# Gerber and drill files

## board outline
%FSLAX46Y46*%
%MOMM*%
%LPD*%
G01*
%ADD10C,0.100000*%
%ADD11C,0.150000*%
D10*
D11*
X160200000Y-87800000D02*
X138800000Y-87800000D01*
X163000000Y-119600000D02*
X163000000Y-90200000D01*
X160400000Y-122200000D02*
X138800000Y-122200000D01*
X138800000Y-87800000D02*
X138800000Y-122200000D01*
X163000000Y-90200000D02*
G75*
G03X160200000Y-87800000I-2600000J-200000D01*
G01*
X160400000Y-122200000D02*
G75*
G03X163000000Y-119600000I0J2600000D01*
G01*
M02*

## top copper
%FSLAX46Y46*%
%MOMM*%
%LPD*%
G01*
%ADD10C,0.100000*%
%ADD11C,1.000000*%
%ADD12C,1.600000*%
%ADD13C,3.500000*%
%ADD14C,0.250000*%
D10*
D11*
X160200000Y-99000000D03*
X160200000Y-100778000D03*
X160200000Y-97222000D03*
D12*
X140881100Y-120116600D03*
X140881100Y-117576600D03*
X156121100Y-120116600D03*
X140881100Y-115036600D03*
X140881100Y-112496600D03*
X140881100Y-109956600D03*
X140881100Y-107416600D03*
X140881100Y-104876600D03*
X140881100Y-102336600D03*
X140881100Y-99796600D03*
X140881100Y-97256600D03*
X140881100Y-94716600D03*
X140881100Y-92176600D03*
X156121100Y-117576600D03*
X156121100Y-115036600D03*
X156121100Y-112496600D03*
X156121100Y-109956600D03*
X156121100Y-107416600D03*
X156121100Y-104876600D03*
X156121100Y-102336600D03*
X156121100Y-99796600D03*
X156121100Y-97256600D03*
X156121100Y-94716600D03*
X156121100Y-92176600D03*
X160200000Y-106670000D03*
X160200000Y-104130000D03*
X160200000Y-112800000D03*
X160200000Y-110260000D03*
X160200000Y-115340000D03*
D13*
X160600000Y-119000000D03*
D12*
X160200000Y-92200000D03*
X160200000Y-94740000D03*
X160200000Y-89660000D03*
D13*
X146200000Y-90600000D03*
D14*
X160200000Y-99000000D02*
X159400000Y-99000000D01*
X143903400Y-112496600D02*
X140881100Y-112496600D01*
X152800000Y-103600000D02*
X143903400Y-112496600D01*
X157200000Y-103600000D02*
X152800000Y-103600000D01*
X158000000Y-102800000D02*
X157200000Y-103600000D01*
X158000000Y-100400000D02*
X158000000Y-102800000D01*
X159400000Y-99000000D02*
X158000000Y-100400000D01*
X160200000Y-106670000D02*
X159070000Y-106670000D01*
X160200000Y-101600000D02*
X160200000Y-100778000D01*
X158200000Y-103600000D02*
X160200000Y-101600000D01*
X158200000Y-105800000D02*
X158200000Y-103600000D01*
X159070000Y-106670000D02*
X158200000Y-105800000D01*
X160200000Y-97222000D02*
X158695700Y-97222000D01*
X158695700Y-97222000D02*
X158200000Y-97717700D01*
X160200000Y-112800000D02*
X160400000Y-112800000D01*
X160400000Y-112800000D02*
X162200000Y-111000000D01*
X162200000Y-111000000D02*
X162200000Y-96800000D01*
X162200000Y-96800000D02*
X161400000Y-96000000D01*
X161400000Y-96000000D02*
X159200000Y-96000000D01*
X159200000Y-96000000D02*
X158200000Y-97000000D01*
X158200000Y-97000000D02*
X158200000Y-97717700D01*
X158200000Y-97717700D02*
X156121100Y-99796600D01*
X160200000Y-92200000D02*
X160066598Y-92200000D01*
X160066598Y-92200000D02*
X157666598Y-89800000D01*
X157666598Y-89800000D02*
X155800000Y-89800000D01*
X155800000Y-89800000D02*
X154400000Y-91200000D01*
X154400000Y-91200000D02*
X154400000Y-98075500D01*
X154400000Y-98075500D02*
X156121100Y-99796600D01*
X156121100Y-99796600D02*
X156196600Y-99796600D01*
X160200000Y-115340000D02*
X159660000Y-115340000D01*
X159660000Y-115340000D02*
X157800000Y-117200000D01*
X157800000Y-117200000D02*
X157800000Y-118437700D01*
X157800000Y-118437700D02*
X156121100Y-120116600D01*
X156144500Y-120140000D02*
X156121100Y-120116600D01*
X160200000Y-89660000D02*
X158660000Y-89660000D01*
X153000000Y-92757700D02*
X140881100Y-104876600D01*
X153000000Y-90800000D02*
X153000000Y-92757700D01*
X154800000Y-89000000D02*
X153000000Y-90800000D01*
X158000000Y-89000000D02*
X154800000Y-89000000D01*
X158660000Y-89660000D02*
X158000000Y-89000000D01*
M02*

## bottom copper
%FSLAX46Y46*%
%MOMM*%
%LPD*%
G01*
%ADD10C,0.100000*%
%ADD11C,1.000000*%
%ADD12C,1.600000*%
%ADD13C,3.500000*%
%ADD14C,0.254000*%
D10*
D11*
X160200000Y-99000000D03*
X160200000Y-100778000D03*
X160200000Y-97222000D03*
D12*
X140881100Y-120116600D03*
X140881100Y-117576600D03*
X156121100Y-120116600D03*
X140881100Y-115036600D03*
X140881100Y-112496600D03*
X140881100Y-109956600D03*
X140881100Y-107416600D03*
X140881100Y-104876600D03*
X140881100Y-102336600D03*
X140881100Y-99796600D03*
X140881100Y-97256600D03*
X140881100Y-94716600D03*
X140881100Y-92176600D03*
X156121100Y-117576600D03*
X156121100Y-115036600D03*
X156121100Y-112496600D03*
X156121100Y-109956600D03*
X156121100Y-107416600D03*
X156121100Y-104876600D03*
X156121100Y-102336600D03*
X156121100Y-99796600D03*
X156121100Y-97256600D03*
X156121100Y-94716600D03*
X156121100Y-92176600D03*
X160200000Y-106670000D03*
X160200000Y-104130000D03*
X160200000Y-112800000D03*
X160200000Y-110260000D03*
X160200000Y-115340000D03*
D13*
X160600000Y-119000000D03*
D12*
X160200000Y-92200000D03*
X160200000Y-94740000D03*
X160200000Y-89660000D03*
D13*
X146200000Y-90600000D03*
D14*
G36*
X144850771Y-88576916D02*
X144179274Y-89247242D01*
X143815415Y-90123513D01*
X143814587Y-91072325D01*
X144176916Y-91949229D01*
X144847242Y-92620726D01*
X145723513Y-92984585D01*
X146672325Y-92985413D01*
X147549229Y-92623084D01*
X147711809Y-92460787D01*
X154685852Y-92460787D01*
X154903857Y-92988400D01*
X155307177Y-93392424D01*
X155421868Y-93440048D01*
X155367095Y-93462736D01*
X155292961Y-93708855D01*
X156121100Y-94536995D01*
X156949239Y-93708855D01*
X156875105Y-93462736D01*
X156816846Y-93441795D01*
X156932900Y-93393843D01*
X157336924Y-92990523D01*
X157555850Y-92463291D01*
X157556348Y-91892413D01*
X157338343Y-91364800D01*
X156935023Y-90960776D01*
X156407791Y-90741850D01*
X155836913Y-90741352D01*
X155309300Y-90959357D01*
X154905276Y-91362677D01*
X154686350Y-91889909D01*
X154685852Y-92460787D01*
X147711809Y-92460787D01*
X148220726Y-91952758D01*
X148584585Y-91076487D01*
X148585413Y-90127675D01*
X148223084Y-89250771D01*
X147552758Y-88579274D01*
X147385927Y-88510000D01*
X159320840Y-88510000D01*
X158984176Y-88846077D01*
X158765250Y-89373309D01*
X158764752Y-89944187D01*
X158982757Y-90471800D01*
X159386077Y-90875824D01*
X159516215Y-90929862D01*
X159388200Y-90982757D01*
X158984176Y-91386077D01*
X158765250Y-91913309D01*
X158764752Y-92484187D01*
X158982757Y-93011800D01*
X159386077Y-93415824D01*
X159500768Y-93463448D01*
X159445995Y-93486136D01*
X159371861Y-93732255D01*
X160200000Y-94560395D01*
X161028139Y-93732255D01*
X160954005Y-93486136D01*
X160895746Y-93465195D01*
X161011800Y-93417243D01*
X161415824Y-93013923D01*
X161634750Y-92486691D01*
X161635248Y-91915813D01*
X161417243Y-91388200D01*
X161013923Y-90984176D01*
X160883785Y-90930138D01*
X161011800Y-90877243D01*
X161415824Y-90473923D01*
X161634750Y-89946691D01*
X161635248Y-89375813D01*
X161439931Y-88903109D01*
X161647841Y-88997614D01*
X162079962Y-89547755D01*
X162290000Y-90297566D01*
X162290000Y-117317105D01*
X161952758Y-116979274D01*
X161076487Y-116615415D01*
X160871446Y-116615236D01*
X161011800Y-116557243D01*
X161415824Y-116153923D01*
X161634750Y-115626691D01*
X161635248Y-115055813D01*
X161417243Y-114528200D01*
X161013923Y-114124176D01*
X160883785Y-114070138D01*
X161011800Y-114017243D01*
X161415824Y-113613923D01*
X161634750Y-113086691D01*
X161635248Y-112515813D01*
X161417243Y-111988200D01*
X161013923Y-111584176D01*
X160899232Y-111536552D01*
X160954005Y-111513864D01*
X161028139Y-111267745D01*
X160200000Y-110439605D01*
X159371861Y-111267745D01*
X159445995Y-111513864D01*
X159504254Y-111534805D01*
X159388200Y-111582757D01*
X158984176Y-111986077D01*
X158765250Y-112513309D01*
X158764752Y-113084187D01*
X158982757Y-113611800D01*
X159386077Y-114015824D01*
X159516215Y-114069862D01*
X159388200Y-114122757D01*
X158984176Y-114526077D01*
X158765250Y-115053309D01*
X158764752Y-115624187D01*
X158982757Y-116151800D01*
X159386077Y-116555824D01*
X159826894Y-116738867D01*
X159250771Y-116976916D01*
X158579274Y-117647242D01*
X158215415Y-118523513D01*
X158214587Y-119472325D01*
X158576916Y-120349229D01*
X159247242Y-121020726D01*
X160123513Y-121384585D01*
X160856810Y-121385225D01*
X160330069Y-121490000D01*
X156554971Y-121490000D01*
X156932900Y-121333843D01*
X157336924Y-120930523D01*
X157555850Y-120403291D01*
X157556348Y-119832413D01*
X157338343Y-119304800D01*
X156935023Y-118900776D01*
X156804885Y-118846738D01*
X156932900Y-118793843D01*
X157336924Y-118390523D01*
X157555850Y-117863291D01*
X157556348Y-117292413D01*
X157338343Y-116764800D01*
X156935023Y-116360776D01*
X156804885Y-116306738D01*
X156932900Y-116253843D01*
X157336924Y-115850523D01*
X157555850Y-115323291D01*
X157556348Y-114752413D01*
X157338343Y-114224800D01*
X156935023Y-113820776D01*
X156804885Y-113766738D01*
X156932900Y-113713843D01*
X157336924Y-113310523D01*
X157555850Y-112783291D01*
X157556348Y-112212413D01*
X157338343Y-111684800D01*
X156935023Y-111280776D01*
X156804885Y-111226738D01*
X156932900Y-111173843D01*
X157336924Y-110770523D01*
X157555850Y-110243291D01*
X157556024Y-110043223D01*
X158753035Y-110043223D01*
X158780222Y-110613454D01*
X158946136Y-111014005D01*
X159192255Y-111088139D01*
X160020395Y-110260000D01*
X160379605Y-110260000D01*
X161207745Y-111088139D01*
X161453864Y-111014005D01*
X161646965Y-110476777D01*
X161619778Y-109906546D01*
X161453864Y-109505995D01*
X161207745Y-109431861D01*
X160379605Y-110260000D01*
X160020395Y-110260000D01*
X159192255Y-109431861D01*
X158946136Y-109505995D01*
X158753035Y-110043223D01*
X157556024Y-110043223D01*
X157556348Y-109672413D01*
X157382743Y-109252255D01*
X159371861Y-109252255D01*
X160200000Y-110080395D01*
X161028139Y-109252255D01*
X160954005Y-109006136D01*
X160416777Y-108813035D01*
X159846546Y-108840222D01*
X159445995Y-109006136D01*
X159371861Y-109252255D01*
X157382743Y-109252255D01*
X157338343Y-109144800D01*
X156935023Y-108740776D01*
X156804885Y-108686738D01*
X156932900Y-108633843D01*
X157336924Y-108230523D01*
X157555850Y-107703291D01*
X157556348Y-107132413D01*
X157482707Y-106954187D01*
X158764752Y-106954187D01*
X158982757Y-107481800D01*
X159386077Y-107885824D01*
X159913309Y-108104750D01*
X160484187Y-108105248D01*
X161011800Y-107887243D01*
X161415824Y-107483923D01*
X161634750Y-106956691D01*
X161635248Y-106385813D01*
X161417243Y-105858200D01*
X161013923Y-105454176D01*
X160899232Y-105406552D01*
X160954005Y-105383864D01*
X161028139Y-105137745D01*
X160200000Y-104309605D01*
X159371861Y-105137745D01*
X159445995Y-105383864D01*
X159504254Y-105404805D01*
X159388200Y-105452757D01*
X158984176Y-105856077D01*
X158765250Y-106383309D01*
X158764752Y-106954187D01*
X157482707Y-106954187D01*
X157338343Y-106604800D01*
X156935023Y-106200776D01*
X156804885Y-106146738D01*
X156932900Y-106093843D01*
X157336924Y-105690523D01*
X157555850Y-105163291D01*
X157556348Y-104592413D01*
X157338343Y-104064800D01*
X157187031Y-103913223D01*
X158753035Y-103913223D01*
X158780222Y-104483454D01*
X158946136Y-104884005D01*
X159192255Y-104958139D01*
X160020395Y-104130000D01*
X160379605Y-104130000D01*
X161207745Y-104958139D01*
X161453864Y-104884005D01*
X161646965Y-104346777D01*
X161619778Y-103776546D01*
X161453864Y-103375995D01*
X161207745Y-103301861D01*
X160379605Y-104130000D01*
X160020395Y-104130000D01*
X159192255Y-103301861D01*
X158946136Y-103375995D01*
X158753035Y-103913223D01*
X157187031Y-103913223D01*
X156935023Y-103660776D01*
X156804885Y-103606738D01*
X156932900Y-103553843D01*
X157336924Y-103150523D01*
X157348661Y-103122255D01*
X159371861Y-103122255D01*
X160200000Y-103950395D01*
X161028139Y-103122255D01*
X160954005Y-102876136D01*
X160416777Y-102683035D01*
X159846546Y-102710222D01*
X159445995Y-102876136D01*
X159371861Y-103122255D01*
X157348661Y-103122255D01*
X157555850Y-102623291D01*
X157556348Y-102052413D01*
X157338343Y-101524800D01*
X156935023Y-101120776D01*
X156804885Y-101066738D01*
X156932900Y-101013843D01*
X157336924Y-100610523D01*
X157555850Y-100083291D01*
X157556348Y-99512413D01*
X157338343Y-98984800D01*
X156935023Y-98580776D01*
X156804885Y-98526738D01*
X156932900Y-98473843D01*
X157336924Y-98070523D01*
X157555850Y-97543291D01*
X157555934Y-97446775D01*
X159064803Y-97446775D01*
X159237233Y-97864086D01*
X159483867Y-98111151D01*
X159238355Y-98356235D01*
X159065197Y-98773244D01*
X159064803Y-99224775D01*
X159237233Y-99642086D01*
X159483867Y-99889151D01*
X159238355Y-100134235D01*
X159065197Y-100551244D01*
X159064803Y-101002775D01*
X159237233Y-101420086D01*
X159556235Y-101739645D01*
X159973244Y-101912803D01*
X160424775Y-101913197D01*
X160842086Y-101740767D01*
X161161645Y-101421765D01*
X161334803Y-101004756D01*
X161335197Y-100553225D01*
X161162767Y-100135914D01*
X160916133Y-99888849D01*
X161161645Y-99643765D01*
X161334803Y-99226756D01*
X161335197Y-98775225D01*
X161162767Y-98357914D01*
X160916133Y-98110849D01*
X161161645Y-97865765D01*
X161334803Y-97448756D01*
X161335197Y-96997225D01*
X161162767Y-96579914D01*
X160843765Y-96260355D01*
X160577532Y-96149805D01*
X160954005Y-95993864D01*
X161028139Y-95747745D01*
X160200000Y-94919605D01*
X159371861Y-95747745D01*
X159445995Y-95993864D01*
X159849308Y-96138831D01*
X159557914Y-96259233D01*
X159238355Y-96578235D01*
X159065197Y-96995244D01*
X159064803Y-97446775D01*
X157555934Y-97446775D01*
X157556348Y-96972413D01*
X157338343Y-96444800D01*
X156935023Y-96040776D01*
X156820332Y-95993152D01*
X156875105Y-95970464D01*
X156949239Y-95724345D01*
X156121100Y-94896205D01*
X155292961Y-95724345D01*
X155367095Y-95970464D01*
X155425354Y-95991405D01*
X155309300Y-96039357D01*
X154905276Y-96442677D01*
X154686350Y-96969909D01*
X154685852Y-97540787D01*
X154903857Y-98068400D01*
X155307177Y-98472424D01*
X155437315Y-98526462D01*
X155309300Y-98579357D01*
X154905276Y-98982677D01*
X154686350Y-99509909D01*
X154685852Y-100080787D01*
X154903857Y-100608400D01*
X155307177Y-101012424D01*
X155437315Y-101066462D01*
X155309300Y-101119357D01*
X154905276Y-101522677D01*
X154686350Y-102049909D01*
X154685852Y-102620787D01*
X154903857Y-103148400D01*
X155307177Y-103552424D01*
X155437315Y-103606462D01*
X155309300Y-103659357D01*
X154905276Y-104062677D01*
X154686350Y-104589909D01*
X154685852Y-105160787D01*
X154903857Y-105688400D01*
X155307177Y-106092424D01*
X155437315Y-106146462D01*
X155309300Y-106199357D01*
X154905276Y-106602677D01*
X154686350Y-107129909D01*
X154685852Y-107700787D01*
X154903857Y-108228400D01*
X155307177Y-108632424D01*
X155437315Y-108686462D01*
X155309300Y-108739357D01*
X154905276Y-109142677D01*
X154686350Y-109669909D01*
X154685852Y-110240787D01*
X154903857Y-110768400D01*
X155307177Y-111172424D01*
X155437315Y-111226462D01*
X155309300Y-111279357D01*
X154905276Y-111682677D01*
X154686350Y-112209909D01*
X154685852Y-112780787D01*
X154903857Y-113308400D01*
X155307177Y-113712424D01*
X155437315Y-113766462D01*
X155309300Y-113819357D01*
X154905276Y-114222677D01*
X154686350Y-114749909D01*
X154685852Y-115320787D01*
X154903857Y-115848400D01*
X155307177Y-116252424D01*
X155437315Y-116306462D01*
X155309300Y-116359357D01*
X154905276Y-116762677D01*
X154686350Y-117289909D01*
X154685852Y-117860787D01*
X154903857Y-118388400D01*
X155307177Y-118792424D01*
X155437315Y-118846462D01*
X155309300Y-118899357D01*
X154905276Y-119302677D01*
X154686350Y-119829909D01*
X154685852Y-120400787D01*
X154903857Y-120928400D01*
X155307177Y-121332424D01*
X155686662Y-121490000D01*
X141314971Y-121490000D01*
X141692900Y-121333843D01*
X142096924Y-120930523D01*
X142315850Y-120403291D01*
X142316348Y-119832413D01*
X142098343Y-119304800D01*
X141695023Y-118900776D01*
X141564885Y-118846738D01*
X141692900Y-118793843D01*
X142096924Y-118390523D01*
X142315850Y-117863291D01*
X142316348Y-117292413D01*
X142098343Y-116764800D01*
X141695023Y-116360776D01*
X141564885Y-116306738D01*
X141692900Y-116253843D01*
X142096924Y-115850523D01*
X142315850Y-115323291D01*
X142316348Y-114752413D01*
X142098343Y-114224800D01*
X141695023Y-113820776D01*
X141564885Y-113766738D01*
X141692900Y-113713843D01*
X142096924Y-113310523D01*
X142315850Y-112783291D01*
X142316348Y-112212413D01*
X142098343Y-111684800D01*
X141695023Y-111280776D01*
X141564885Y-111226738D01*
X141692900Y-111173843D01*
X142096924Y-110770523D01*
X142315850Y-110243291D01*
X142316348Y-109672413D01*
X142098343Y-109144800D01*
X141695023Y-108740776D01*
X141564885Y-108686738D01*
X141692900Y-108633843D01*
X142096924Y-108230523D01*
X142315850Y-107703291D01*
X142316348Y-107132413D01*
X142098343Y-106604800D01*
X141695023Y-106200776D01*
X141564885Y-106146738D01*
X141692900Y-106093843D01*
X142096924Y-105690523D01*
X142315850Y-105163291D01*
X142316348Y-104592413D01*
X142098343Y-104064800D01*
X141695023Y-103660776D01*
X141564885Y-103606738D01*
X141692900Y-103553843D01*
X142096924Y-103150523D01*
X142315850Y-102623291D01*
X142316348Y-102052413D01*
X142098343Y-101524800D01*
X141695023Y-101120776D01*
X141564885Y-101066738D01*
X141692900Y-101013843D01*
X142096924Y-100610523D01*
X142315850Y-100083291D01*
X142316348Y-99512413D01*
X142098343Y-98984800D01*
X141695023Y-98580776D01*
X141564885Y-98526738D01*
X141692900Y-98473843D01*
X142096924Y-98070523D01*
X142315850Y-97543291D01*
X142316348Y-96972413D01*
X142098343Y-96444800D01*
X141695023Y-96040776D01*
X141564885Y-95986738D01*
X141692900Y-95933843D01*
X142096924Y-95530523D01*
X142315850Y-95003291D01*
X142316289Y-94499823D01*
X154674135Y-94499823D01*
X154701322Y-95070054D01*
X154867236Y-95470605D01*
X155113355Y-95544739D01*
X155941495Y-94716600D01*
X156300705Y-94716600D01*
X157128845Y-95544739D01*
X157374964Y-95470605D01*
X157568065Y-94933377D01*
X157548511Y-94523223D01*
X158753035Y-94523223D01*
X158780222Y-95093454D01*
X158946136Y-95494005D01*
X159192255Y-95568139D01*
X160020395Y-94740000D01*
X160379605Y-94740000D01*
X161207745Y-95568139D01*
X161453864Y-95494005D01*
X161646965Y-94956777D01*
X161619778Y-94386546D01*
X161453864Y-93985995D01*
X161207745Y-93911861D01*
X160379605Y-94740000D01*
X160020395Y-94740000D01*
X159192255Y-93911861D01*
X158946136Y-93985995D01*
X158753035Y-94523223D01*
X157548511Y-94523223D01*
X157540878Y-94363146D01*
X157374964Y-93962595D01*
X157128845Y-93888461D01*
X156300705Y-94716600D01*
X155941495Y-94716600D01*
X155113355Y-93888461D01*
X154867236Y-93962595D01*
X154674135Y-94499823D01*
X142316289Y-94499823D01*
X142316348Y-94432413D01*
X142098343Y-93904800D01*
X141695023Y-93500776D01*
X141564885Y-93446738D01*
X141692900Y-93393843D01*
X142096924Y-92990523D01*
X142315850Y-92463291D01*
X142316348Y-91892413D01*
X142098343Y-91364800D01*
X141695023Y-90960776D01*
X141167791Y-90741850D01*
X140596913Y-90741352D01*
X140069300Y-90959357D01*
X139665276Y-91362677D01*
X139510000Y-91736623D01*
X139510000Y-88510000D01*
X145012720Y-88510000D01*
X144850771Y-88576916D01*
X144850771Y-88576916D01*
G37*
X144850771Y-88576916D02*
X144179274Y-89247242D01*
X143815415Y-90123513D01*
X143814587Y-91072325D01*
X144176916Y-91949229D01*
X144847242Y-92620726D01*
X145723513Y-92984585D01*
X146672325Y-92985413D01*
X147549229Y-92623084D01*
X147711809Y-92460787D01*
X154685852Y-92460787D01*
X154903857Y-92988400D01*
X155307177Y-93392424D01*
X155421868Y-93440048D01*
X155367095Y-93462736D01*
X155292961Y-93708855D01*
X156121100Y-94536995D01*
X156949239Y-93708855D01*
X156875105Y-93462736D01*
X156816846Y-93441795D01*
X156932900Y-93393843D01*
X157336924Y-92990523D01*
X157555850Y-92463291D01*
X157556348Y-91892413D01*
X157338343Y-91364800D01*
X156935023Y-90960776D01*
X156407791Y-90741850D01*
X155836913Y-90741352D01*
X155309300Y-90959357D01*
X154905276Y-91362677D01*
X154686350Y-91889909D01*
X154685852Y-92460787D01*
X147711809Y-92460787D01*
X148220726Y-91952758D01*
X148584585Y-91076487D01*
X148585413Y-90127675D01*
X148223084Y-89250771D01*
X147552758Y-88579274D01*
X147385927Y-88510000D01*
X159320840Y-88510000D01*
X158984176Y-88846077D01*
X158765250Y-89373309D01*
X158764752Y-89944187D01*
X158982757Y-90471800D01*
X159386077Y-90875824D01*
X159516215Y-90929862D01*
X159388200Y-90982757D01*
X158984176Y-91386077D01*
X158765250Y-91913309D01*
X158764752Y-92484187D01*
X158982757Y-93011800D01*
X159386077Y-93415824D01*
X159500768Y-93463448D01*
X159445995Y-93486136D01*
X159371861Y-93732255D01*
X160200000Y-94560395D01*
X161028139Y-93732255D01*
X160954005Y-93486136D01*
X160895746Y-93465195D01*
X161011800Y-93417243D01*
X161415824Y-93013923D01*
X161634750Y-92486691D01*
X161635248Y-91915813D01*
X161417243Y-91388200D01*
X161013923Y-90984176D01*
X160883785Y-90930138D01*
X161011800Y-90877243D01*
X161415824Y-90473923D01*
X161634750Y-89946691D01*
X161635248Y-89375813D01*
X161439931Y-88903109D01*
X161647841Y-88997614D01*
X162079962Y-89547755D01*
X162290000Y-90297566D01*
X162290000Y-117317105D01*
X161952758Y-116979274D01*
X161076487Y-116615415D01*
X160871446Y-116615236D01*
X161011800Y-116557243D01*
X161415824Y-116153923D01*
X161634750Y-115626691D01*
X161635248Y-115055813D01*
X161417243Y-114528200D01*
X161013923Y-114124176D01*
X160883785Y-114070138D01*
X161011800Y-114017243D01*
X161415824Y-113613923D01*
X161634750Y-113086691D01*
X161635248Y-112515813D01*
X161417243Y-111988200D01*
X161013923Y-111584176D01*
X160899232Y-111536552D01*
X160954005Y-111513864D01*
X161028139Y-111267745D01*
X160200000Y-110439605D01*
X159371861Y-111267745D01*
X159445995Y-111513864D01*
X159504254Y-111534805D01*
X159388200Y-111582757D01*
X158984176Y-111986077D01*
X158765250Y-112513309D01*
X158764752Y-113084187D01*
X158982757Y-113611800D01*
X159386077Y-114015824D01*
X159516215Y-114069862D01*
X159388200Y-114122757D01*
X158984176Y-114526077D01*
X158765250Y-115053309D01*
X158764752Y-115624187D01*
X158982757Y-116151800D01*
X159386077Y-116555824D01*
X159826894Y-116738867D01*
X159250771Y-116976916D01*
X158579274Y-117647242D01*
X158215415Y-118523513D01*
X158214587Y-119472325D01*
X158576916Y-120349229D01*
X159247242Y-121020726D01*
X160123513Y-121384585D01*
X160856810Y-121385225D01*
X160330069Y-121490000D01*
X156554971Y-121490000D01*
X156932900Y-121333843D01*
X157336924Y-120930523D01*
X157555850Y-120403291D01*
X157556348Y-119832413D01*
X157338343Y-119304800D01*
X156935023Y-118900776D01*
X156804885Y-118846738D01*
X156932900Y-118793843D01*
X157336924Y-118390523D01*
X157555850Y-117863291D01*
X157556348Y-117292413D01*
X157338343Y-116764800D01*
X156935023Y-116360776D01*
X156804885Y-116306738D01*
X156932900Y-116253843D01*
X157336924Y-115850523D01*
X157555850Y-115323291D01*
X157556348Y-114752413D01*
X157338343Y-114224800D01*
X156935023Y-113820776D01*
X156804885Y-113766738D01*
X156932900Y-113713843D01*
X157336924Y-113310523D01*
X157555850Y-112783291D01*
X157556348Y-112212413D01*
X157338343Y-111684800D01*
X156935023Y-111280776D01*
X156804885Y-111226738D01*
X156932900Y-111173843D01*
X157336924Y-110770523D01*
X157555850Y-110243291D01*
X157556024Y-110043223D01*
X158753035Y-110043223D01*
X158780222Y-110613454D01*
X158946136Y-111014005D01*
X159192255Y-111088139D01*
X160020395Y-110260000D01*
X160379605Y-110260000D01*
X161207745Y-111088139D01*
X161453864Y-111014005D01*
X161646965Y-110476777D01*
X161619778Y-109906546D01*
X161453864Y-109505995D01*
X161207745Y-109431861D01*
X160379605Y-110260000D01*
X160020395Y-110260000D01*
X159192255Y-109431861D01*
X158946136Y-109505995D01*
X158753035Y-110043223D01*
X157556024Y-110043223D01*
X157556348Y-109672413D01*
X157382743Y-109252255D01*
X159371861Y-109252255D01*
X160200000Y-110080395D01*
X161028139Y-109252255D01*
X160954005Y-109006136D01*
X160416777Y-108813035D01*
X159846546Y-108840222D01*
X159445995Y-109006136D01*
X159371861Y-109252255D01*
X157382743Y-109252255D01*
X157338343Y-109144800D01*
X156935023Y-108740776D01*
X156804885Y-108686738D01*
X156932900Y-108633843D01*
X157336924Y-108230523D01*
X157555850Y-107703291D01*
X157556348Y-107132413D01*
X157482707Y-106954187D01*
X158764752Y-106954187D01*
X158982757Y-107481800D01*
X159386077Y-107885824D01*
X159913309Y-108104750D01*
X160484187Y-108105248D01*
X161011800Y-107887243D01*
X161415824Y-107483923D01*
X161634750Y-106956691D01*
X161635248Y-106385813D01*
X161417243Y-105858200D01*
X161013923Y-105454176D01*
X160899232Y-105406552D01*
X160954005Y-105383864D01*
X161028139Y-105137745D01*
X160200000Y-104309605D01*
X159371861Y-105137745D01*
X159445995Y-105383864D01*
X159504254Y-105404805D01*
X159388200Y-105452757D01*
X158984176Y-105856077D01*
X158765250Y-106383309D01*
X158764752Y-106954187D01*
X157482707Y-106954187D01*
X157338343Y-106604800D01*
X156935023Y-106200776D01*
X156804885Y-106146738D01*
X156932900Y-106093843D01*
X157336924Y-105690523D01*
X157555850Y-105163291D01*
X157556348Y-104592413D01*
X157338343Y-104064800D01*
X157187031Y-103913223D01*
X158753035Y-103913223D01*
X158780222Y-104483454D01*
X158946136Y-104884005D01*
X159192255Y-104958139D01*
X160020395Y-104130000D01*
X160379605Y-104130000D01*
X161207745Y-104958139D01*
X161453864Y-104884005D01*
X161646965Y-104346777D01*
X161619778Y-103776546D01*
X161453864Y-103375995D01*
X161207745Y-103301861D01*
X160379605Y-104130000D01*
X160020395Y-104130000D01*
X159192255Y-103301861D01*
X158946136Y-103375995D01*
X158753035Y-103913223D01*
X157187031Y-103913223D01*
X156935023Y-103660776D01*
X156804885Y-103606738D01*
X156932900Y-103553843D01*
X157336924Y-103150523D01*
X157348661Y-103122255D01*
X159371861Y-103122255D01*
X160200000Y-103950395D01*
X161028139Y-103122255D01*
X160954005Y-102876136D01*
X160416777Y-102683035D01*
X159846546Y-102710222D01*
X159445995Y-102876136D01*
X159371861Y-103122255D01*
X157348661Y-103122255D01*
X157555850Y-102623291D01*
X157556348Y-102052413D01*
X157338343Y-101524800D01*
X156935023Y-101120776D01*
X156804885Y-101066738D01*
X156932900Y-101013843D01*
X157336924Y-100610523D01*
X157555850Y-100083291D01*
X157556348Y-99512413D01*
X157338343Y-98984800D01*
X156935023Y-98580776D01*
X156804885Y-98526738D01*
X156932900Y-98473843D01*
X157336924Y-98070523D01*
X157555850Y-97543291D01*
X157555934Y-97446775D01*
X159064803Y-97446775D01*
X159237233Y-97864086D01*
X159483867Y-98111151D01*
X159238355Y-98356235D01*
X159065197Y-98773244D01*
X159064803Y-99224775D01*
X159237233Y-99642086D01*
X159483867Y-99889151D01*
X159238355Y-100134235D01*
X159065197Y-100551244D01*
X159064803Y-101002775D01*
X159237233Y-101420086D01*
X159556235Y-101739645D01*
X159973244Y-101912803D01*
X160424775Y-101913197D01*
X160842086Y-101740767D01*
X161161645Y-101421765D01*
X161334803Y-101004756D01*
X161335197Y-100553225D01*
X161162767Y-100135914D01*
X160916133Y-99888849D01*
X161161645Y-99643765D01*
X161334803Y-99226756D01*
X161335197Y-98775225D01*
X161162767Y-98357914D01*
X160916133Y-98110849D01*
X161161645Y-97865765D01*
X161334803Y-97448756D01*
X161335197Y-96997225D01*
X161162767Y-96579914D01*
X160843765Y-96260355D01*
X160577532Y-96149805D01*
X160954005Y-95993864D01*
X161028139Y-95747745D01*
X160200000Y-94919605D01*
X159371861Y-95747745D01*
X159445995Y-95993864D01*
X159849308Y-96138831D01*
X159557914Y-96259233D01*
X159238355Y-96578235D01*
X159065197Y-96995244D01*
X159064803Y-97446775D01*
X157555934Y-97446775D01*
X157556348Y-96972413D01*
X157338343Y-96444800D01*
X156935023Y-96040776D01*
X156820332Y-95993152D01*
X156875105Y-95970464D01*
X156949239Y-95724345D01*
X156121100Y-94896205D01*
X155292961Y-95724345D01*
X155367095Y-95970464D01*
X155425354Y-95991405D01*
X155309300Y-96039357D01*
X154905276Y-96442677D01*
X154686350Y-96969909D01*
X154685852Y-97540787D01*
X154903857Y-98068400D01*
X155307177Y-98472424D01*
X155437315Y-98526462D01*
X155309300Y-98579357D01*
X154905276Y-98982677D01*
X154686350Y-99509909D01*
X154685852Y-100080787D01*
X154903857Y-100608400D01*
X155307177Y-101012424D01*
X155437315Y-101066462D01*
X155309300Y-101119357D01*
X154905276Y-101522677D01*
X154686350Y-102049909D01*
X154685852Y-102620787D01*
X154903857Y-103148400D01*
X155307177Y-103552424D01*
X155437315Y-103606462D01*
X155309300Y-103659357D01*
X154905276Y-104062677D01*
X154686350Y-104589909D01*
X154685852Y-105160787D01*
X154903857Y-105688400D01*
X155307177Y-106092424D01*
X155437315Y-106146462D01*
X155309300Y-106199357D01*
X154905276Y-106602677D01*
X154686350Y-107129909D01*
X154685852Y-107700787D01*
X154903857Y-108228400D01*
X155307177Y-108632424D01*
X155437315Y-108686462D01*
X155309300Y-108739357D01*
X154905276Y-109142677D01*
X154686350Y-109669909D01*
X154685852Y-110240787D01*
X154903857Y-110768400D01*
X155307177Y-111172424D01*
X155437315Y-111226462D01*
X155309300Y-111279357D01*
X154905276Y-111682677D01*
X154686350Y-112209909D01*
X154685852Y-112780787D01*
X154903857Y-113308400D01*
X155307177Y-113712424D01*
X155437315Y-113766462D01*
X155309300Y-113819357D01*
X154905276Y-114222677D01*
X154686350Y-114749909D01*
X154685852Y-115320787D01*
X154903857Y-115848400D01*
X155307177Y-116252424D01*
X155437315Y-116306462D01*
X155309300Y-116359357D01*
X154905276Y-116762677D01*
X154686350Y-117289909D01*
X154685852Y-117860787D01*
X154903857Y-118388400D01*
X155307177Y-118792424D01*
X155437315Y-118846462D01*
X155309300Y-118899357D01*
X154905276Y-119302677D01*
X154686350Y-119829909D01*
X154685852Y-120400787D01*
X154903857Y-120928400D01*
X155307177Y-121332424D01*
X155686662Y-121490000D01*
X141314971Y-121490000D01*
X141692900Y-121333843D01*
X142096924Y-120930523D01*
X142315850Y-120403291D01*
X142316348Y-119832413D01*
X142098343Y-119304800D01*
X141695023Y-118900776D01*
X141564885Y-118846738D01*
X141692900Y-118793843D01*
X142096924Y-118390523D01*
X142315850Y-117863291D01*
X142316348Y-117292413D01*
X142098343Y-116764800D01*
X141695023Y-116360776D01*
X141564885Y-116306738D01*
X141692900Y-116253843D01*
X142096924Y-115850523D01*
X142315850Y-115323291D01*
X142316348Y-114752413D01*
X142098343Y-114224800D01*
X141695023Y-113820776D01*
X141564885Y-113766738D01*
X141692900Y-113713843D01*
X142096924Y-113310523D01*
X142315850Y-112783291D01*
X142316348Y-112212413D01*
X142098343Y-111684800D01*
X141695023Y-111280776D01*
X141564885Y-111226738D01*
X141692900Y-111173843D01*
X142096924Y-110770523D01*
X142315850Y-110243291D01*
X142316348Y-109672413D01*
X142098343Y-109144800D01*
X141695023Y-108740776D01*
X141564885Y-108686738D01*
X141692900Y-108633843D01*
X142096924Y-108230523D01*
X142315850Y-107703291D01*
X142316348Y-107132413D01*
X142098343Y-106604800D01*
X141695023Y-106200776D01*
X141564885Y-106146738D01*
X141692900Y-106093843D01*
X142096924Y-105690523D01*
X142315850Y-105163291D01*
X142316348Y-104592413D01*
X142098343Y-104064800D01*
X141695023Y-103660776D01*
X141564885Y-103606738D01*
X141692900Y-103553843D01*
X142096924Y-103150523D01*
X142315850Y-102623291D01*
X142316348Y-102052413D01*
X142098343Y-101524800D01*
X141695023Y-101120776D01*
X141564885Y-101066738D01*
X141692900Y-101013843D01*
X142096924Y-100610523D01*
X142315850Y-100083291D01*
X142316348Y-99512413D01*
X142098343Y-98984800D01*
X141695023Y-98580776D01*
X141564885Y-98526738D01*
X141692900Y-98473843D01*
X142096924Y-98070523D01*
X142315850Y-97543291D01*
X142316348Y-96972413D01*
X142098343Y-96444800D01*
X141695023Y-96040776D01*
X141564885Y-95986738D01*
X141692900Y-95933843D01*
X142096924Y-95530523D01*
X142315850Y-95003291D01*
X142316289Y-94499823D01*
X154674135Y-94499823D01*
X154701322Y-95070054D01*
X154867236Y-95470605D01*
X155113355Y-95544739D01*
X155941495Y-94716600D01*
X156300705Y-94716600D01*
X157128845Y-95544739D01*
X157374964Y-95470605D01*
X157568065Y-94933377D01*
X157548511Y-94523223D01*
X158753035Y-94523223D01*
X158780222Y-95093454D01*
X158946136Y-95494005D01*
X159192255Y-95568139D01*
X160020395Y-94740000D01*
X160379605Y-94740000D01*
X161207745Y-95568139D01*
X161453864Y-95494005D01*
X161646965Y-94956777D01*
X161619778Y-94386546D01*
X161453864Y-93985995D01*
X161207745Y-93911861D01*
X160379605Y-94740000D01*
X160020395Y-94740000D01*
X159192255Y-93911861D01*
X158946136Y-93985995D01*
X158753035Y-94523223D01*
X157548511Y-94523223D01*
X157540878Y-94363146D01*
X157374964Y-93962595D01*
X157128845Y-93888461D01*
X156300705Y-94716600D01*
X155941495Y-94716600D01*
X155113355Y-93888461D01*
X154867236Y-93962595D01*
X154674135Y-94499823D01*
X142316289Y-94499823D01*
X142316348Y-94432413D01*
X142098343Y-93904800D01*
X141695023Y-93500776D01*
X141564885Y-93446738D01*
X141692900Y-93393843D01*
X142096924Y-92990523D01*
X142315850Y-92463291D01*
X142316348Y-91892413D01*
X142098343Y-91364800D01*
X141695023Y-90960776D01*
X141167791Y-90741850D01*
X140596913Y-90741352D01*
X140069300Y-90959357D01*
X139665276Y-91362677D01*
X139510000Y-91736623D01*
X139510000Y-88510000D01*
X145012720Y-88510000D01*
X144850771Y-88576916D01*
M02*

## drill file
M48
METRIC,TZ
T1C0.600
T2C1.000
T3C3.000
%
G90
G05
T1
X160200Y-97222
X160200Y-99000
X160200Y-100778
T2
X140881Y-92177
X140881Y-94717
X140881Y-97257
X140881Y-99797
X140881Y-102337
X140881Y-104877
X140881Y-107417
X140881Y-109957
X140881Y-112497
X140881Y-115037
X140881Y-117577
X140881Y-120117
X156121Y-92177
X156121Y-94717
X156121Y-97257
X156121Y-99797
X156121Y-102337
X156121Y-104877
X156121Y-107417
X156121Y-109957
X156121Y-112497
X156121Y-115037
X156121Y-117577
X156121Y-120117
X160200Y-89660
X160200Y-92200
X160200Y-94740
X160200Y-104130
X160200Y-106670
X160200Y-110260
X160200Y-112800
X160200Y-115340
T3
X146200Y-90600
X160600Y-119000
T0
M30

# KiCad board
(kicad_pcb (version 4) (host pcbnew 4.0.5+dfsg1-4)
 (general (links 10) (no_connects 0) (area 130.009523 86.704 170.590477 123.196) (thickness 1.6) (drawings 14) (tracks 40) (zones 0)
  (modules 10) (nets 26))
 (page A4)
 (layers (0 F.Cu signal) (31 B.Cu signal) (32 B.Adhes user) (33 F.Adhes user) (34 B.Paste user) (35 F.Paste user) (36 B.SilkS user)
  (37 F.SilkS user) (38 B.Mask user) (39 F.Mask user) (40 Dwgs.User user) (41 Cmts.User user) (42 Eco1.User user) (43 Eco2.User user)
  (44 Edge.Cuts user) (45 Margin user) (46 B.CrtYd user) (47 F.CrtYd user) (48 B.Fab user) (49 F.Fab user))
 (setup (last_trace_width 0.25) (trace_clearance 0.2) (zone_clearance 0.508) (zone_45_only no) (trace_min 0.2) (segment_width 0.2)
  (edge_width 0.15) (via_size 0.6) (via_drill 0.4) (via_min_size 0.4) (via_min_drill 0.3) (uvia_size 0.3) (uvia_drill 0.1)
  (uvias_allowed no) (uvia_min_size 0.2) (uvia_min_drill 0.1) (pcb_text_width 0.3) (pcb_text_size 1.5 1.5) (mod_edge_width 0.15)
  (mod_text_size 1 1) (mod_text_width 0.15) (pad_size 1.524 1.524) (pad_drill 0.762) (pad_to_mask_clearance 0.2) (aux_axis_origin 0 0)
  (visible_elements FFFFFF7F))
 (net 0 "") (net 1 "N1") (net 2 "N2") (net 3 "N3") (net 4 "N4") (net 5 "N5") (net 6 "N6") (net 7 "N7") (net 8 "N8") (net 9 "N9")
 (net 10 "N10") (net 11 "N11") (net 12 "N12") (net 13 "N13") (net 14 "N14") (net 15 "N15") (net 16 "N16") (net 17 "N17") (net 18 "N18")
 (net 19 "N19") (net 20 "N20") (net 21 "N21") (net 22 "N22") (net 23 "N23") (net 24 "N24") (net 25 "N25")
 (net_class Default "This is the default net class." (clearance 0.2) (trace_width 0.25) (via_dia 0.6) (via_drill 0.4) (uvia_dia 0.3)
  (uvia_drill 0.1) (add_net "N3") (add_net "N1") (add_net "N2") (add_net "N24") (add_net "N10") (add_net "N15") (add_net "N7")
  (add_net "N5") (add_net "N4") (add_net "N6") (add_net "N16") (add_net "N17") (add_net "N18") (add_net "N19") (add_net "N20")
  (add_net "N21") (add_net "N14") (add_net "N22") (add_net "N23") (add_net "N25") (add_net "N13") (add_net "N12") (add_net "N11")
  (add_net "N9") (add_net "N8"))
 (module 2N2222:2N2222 (layer F.Cu) (at 160.2 99 270)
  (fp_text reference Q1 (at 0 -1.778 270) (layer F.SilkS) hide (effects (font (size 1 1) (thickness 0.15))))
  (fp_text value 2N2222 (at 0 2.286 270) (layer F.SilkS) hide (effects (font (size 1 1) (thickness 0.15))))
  (pad 2 thru_hole circle (at 0 0 270) (size 1 1) (drill 0.6) (layers *.Cu *.Mask F.SilkS) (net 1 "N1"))
  (pad 3 thru_hole circle (at 1.778 0 270) (size 1 1) (drill 0.6) (layers *.Cu *.Mask F.SilkS) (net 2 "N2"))
  (pad 1 thru_hole circle (at -1.778 0 270) (size 1 1) (drill 0.6) (layers *.Cu *.Mask F.SilkS) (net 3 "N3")))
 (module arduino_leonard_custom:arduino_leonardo (layer F.Cu) (at 148.5011 105.0036)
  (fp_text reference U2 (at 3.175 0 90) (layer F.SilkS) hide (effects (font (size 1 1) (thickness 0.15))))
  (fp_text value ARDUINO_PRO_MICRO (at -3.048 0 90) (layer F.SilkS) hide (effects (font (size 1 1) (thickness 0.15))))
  (pad 12 thru_hole circle (at -7.62 15.113) (size 1.6 1.6) (drill 1) (layers *.Cu *.Mask F.SilkS) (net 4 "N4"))
  (pad 11 thru_hole circle (at -7.62 12.573) (size 1.6 1.6) (drill 1) (layers *.Cu *.Mask F.SilkS) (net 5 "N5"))
  (pad 13 thru_hole circle (at 7.62 15.113) (size 1.6 1.6) (drill 1) (layers *.Cu *.Mask F.SilkS) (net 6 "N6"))
  (pad 10 thru_hole circle (at -7.62 10.033) (size 1.6 1.6) (drill 1) (layers *.Cu *.Mask F.SilkS) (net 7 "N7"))
  (pad 9 thru_hole circle (at -7.62 7.493) (size 1.6 1.6) (drill 1) (layers *.Cu *.Mask F.SilkS) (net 1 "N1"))
  (pad 8 thru_hole circle (at -7.62 4.953) (size 1.6 1.6) (drill 1) (layers *.Cu *.Mask F.SilkS) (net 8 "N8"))
  (pad 7 thru_hole circle (at -7.62 2.413) (size 1.6 1.6) (drill 1) (layers *.Cu *.Mask F.SilkS) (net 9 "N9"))
  (pad 6 thru_hole circle (at -7.62 -0.127) (size 1.6 1.6) (drill 1) (layers *.Cu *.Mask F.SilkS) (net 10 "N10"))
  (pad 5 thru_hole circle (at -7.62 -2.667) (size 1.6 1.6) (drill 1) (layers *.Cu *.Mask F.SilkS) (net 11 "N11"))
  (pad 4 thru_hole circle (at -7.62 -5.207) (size 1.6 1.6) (drill 1) (layers *.Cu *.Mask F.SilkS) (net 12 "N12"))
  (pad 3 thru_hole circle (at -7.62 -7.747) (size 1.6 1.6) (drill 1) (layers *.Cu *.Mask F.SilkS) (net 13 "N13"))
  (pad 2 thru_hole circle (at -7.62 -10.287) (size 1.6 1.6) (drill 1) (layers *.Cu *.Mask F.SilkS) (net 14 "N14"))
  (pad 1 thru_hole circle (at -7.62 -12.827) (size 1.6 1.6) (drill 1) (layers *.Cu *.Mask F.SilkS) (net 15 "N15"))
  (pad 14 thru_hole circle (at 7.62 12.573) (size 1.6 1.6) (drill 1) (layers *.Cu *.Mask F.SilkS) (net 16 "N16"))
  (pad 15 thru_hole circle (at 7.62 10.033) (size 1.6 1.6) (drill 1) (layers *.Cu *.Mask F.SilkS) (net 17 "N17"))
  (pad 16 thru_hole circle (at 7.62 7.493) (size 1.6 1.6) (drill 1) (layers *.Cu *.Mask F.SilkS) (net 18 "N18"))
  (pad 17 thru_hole circle (at 7.62 4.953) (size 1.6 1.6) (drill 1) (layers *.Cu *.Mask F.SilkS) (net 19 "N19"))
  (pad 18 thru_hole circle (at 7.62 2.413) (size 1.6 1.6) (drill 1) (layers *.Cu *.Mask F.SilkS) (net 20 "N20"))
  (pad 19 thru_hole circle (at 7.62 -0.127) (size 1.6 1.6) (drill 1) (layers *.Cu *.Mask F.SilkS) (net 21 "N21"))
  (pad 20 thru_hole circle (at 7.62 -2.667) (size 1.6 1.6) (drill 1) (layers *.Cu *.Mask F.SilkS) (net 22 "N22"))
  (pad 21 thru_hole circle (at 7.62 -5.207) (size 1.6 1.6) (drill 1) (layers *.Cu *.Mask F.SilkS) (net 3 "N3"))
  (pad 22 thru_hole circle (at 7.62 -7.747) (size 1.6 1.6) (drill 1) (layers *.Cu *.Mask F.SilkS) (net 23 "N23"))
  (pad 23 thru_hole circle (at 7.62 -10.287) (size 1.6 1.6) (drill 1) (layers *.Cu *.Mask F.SilkS) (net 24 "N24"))
  (pad 24 thru_hole circle (at 7.62 -12.827) (size 1.6 1.6) (drill 1) (layers *.Cu *.Mask F.SilkS) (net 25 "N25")))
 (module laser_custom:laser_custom (layer F.Cu) (at 160.2 105.4 90)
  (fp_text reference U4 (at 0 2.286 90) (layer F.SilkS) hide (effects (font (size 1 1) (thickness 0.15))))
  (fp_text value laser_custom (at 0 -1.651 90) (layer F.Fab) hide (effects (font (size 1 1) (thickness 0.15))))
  (pad 1 thru_hole circle (at -1.27 0 90) (size 1.6 1.6) (drill 1) (layers *.Cu *.Mask) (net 2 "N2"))
  (pad 2 thru_hole circle (at 1.27 0 90) (size 1.6 1.6) (drill 1) (layers *.Cu *.Mask) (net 24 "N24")))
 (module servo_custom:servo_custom (layer F.Cu) (at 160.2 112.8 270)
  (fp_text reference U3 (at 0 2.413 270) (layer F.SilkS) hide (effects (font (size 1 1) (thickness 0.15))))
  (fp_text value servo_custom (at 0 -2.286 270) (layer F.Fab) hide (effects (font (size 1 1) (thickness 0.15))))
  (pad 2 thru_hole circle (at 0 0 270) (size 1.6 1.6) (drill 1) (layers *.Cu *.Mask) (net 3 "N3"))
  (pad 1 thru_hole circle (at -2.54 0 270) (size 1.6 1.6) (drill 1) (layers *.Cu *.Mask) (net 24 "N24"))
  (pad 3 thru_hole circle (at 2.54 0 270) (size 1.6 1.6) (drill 1) (layers *.Cu *.Mask) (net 6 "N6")))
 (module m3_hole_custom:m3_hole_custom (layer F.Cu) (at 136.4 119.2)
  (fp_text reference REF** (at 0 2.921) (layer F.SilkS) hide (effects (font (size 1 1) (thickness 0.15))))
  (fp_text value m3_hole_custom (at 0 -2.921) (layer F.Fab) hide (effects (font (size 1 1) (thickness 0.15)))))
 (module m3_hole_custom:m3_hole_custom (layer F.Cu) (at 164.2 90.6)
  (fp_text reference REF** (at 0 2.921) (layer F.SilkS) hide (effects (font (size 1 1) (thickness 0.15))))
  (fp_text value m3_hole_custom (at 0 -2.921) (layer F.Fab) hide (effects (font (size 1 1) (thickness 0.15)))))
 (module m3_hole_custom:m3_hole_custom (layer F.Cu) (at 136.4 90.6)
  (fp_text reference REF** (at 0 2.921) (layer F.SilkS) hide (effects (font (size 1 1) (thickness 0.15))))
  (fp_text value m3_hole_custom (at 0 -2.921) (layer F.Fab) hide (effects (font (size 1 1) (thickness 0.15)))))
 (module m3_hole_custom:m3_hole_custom (layer F.Cu) (at 160.6 119)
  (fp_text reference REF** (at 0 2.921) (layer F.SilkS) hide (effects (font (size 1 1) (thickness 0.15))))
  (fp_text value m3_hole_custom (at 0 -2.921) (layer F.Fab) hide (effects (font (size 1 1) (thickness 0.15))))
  (pad 1 thru_hole circle (at 0 0) (size 3.5 3.5) (drill 3) (layers *.Cu *.Mask)))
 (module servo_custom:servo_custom (layer F.Cu) (at 160.2 92.2 90)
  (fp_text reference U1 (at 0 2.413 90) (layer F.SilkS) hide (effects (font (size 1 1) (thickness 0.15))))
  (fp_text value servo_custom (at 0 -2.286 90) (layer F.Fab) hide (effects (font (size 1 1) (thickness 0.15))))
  (pad 2 thru_hole circle (at 0 0 90) (size 1.6 1.6) (drill 1) (layers *.Cu *.Mask) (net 3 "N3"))
  (pad 1 thru_hole circle (at -2.54 0 90) (size 1.6 1.6) (drill 1) (layers *.Cu *.Mask) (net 24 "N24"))
  (pad 3 thru_hole circle (at 2.54 0 90) (size 1.6 1.6) (drill 1) (layers *.Cu *.Mask) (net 10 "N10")))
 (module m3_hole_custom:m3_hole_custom (layer F.Cu) (at 146.2 90.6)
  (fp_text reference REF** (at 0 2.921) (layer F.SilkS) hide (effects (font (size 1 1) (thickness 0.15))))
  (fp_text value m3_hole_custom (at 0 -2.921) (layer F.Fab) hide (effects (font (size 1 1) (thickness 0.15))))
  (pad 1 thru_hole circle (at 0 0) (size 3.5 3.5) (drill 3) (layers *.Cu *.Mask)))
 (gr_line (start 160.2 87.8) (end 138.8 87.8) (angle 90) (layer Edge.Cuts) (width 0.15))
 (gr_line (start 163 119.6) (end 163 90.2) (angle 90) (layer Edge.Cuts) (width 0.15))
 (gr_line (start 160.4 122.2) (end 138.8 122.2) (angle 90) (layer Edge.Cuts) (width 0.15))
 (gr_line (start 138.8 87.8) (end 138.8 122.2) (angle 90) (layer Edge.Cuts) (width 0.15))
 (gr_arc (start 160.4 90.4) (end 160.2 87.8) (angle 90) (layer Edge.Cuts) (width 0.15))
 (gr_arc (start 160.4 119.6) (end 163 119.6) (angle 90) (layer Edge.Cuts) (width 0.15))
 (segment (start 160.2 99) (end 159.4 99) (width 0.25) (layer F.Cu) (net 1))
 (segment (start 143.9034 112.4966) (end 140.8811 112.4966) (width 0.25) (layer F.Cu) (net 1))
 (segment (start 152.8 103.6) (end 143.9034 112.4966) (width 0.25) (layer F.Cu) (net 1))
 (segment (start 157.2 103.6) (end 152.8 103.6) (width 0.25) (layer F.Cu) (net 1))
 (segment (start 158 102.8) (end 157.2 103.6) (width 0.25) (layer F.Cu) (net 1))
 (segment (start 158 100.4) (end 158 102.8) (width 0.25) (layer F.Cu) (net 1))
 (segment (start 159.4 99) (end 158 100.4) (width 0.25) (layer F.Cu) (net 1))
 (segment (start 160.2 106.67) (end 159.07 106.67) (width 0.25) (layer F.Cu) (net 2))
 (segment (start 160.2 101.6) (end 160.2 100.778) (width 0.25) (layer F.Cu) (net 2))
 (segment (start 158.2 103.6) (end 160.2 101.6) (width 0.25) (layer F.Cu) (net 2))
 (segment (start 158.2 105.8) (end 158.2 103.6) (width 0.25) (layer F.Cu) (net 2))
 (segment (start 159.07 106.67) (end 158.2 105.8) (width 0.25) (layer F.Cu) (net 2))
 (segment (start 160.2 97.222) (end 158.6957 97.222) (width 0.25) (layer F.Cu) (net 3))
 (segment (start 158.6957 97.222) (end 158.2 97.7177) (width 0.25) (layer F.Cu) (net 3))
 (segment (start 160.2 112.8) (end 160.4 112.8) (width 0.25) (layer F.Cu) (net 3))
 (segment (start 160.4 112.8) (end 162.2 111) (width 0.25) (layer F.Cu) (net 3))
 (segment (start 162.2 111) (end 162.2 96.8) (width 0.25) (layer F.Cu) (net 3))
 (segment (start 162.2 96.8) (end 161.4 96) (width 0.25) (layer F.Cu) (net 3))
 (segment (start 161.4 96) (end 159.2 96) (width 0.25) (layer F.Cu) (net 3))
 (segment (start 159.2 96) (end 158.2 97) (width 0.25) (layer F.Cu) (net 3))
 (segment (start 158.2 97) (end 158.2 97.7177) (width 0.25) (layer F.Cu) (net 3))
 (segment (start 158.2 97.7177) (end 156.1211 99.7966) (width 0.25) (layer F.Cu) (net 3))
 (segment (start 160.2 92.2) (end 160.066598 92.2) (width 0.25) (layer F.Cu) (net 3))
 (segment (start 160.066598 92.2) (end 157.666598 89.8) (width 0.25) (layer F.Cu) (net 3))
 (segment (start 157.666598 89.8) (end 155.8 89.8) (width 0.25) (layer F.Cu) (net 3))
 (segment (start 155.8 89.8) (end 154.4 91.2) (width 0.25) (layer F.Cu) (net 3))
 (segment (start 154.4 91.2) (end 154.4 98.0755) (width 0.25) (layer F.Cu) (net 3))
 (segment (start 154.4 98.0755) (end 156.1211 99.7966) (width 0.25) (layer F.Cu) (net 3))
 (segment (start 156.1211 99.7966) (end 156.1966 99.7966) (width 0.25) (layer F.Cu) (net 3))
 (segment (start 160.2 115.34) (end 159.66 115.34) (width 0.25) (layer F.Cu) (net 6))
 (segment (start 159.66 115.34) (end 157.8 117.2) (width 0.25) (layer F.Cu) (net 6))
 (segment (start 157.8 117.2) (end 157.8 118.4377) (width 0.25) (layer F.Cu) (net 6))
 (segment (start 157.8 118.4377) (end 156.1211 120.1166) (width 0.25) (layer F.Cu) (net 6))
 (segment (start 156.1445 120.14) (end 156.1211 120.1166) (width 0.25) (layer F.Cu) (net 6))
 (segment (start 160.2 89.66) (end 158.66 89.66) (width 0.25) (layer F.Cu) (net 10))
 (segment (start 153 92.7577) (end 140.8811 104.8766) (width 0.25) (layer F.Cu) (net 10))
 (segment (start 153 90.8) (end 153 92.7577) (width 0.25) (layer F.Cu) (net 10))
 (segment (start 154.8 89) (end 153 90.8) (width 0.25) (layer F.Cu) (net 10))
 (segment (start 158 89) (end 154.8 89) (width 0.25) (layer F.Cu) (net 10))
 (segment (start 158.66 89.66) (end 158 89) (width 0.25) (layer F.Cu) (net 10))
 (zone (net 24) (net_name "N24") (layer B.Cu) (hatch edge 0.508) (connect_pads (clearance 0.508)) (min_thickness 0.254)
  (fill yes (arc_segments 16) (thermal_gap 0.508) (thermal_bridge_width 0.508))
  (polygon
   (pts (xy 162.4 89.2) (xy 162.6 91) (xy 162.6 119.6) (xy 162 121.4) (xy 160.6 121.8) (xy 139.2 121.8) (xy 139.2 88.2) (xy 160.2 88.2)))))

